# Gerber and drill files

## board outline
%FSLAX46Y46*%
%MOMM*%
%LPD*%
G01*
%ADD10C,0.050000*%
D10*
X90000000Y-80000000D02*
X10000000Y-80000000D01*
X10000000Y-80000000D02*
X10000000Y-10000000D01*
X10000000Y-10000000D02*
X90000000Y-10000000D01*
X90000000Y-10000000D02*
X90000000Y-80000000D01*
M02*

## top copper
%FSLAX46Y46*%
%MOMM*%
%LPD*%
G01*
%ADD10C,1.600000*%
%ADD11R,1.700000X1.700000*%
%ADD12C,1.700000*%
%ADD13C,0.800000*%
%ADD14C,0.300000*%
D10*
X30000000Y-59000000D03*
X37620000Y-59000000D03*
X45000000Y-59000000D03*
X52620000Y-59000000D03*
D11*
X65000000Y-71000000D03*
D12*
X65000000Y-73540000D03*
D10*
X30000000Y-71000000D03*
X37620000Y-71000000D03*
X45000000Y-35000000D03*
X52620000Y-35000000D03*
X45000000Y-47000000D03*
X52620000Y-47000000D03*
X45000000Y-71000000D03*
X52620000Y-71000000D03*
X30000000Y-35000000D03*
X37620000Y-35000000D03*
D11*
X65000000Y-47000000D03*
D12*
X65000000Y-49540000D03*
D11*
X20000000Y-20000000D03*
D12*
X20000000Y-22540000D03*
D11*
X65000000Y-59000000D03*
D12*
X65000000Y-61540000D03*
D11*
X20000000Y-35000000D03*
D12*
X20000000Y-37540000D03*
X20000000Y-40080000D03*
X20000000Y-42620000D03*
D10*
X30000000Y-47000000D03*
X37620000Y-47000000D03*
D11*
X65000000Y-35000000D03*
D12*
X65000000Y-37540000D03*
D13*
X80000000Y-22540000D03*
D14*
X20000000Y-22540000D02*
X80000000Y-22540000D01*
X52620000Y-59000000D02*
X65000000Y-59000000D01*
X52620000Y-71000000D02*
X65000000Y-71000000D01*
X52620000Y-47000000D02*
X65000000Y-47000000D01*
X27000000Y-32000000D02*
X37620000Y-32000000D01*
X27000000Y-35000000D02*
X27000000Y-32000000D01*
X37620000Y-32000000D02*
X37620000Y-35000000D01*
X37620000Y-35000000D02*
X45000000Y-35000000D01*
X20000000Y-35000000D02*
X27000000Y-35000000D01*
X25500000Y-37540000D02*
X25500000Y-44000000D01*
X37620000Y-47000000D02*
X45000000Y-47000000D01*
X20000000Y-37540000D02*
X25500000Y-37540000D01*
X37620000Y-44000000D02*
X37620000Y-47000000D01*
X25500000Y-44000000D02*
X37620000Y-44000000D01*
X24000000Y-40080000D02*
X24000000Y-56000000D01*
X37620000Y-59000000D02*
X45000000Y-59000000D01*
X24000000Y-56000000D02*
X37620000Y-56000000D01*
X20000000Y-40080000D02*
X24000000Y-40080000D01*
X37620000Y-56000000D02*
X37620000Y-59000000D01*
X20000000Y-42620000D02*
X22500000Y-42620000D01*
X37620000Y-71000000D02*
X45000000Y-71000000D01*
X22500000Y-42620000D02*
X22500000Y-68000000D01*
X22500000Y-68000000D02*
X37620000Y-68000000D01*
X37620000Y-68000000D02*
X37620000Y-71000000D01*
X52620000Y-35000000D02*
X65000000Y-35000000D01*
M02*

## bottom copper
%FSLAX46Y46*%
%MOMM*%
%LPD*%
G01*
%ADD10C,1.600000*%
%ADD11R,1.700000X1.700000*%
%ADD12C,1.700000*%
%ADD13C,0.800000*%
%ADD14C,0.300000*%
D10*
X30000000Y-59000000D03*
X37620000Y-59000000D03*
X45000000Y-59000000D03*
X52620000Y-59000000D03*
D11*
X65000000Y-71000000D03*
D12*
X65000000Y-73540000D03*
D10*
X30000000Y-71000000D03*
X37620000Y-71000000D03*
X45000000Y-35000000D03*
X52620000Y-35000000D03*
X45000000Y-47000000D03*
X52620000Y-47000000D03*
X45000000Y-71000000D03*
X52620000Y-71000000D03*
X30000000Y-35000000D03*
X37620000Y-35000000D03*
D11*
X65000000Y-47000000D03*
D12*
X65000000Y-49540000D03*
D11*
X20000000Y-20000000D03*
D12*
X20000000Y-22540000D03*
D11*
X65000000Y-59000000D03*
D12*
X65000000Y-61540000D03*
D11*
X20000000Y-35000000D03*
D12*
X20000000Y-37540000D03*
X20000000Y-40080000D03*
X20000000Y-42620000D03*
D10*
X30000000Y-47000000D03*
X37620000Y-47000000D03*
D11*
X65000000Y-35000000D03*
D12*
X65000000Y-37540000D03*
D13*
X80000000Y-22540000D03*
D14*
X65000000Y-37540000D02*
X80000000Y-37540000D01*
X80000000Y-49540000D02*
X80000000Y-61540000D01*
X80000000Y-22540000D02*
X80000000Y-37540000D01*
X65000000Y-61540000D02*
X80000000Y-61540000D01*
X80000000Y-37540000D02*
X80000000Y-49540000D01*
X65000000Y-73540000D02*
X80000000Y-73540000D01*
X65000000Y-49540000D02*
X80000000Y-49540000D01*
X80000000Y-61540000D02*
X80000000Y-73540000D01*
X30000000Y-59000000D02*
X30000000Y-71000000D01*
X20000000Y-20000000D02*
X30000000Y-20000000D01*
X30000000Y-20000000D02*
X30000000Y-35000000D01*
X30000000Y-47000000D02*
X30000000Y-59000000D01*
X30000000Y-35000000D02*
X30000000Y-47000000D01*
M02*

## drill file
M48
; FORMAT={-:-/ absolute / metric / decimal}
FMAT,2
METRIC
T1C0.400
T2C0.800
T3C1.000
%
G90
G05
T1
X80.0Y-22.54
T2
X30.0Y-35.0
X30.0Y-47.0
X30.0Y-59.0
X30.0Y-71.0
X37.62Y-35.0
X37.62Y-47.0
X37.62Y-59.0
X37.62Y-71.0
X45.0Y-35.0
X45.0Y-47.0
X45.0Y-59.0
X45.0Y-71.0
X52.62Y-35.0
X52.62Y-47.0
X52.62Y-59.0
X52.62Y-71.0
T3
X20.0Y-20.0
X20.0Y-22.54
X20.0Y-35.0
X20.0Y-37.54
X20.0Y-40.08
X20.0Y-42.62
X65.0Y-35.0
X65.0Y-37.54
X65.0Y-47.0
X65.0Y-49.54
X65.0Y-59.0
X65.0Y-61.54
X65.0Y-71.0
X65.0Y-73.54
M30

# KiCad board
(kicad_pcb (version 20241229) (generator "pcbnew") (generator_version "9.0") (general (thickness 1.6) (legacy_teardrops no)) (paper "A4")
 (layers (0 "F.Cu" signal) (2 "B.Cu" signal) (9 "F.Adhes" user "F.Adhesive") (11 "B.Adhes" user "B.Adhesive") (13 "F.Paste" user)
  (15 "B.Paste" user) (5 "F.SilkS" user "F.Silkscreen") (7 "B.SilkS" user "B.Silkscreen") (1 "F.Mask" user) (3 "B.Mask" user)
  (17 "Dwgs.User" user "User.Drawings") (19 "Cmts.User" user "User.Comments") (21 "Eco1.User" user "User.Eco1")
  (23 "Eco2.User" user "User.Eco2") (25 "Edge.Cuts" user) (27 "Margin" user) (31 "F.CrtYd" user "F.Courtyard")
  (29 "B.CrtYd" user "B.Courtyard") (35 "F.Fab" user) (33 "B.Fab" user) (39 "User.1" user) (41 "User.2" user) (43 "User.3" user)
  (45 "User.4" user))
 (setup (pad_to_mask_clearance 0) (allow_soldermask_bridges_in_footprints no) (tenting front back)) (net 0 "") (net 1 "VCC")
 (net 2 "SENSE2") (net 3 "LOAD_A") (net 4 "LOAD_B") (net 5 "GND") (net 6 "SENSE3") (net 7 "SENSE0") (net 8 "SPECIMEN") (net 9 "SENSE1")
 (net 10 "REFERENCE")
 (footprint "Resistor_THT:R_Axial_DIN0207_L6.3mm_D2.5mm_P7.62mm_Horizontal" (layer "F.Cu") (at 30 59)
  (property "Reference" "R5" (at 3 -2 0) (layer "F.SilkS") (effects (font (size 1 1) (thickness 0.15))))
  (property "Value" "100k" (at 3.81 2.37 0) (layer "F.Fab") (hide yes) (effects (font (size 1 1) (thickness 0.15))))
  (pad "1" thru_hole circle (at 0 0) (size 1.6 1.6) (drill 0.8) (layers "*.Cu" "*.Mask") (remove_unused_layers no) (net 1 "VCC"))
  (pad "2" thru_hole circle (at 7.62 0) (size 1.6 1.6) (drill 0.8) (layers "*.Cu" "*.Mask") (remove_unused_layers no) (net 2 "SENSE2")))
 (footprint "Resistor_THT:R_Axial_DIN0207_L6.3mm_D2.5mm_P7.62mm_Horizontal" (layer "F.Cu") (at 45 59)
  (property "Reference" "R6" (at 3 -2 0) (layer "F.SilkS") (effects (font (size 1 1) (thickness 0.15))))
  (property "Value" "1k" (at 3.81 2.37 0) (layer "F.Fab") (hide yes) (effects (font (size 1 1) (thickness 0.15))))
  (pad "1" thru_hole circle (at 0 0) (size 1.6 1.6) (drill 0.8) (layers "*.Cu" "*.Mask") (remove_unused_layers no) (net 2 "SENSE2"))
  (pad "2" thru_hole circle (at 7.62 0) (size 1.6 1.6) (drill 0.8) (layers "*.Cu" "*.Mask") (remove_unused_layers no) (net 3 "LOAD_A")))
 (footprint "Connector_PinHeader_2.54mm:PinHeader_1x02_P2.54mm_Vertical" (layer "F.Cu") (at 65 71)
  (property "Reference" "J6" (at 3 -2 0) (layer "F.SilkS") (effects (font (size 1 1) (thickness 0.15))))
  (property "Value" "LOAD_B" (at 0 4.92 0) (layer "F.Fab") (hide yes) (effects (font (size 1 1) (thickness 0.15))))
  (pad "1" thru_hole rect (at 0 0) (size 1.7 1.7) (drill 1) (layers "*.Cu" "*.Mask") (remove_unused_layers no) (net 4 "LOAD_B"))
  (pad "2" thru_hole circle (at 0 2.54) (size 1.7 1.7) (drill 1) (layers "*.Cu" "*.Mask") (remove_unused_layers no) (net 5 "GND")))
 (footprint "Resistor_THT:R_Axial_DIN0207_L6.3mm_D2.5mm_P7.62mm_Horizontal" (layer "F.Cu") (at 30 71)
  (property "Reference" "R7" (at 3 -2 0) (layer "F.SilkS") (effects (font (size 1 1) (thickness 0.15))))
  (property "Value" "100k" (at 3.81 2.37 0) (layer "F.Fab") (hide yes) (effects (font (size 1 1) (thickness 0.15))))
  (pad "1" thru_hole circle (at 0 0) (size 1.6 1.6) (drill 0.8) (layers "*.Cu" "*.Mask") (remove_unused_layers no) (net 1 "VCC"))
  (pad "2" thru_hole circle (at 7.62 0) (size 1.6 1.6) (drill 0.8) (layers "*.Cu" "*.Mask") (remove_unused_layers no) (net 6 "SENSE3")))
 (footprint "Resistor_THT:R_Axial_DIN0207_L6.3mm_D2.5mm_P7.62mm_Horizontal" (layer "F.Cu") (at 45 35)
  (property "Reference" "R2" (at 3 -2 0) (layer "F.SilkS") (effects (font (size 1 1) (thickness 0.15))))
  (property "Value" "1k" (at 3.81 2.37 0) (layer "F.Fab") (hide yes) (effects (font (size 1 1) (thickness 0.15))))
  (pad "1" thru_hole circle (at 0 0) (size 1.6 1.6) (drill 0.8) (layers "*.Cu" "*.Mask") (remove_unused_layers no) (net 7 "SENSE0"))
  (pad "2" thru_hole circle (at 7.62 0) (size 1.6 1.6) (drill 0.8) (layers "*.Cu" "*.Mask") (remove_unused_layers no) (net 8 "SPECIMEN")))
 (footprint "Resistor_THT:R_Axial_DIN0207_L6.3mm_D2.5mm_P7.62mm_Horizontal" (layer "F.Cu") (at 45 47)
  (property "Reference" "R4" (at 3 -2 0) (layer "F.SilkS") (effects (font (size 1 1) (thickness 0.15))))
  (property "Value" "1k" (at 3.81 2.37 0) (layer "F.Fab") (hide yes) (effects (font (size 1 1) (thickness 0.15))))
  (pad "1" thru_hole circle (at 0 0) (size 1.6 1.6) (drill 0.8) (layers "*.Cu" "*.Mask") (remove_unused_layers no) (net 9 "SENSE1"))
  (pad "2" thru_hole circle (at 7.62 0) (size 1.6 1.6) (drill 0.8) (layers "*.Cu" "*.Mask") (remove_unused_layers no) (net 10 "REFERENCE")))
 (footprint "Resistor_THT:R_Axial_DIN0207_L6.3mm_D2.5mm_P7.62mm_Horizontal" (layer "F.Cu") (at 45 71)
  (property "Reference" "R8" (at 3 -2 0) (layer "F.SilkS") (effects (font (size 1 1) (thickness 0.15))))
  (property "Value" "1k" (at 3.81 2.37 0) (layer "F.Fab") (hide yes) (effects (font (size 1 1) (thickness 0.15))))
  (pad "1" thru_hole circle (at 0 0) (size 1.6 1.6) (drill 0.8) (layers "*.Cu" "*.Mask") (remove_unused_layers no) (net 6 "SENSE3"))
  (pad "2" thru_hole circle (at 7.62 0) (size 1.6 1.6) (drill 0.8) (layers "*.Cu" "*.Mask") (remove_unused_layers no) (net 4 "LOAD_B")))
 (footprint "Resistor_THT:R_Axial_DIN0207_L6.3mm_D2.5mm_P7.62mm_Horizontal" (layer "F.Cu") (at 30 35)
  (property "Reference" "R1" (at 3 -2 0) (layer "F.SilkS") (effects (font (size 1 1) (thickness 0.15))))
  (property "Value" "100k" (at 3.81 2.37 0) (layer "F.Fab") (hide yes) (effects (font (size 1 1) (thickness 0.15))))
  (pad "1" thru_hole circle (at 0 0) (size 1.6 1.6) (drill 0.8) (layers "*.Cu" "*.Mask") (remove_unused_layers no) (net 1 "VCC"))
  (pad "2" thru_hole circle (at 7.62 0) (size 1.6 1.6) (drill 0.8) (layers "*.Cu" "*.Mask") (remove_unused_layers no) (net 7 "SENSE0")))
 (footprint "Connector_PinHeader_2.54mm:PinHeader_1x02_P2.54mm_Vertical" (layer "F.Cu") (at 65 47)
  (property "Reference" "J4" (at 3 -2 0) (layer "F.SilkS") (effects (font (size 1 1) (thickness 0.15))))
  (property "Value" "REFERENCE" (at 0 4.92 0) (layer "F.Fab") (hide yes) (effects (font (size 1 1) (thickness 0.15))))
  (pad "1" thru_hole rect (at 0 0) (size 1.7 1.7) (drill 1) (layers "*.Cu" "*.Mask") (remove_unused_layers no) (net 10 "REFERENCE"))
  (pad "2" thru_hole circle (at 0 2.54) (size 1.7 1.7) (drill 1) (layers "*.Cu" "*.Mask") (remove_unused_layers no) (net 5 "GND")))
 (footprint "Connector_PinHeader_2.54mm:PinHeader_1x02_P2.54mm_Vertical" (layer "F.Cu") (at 20 20)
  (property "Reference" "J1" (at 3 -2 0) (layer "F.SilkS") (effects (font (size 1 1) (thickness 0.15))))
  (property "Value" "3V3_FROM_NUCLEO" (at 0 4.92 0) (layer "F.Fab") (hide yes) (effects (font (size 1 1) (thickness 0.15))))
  (pad "1" thru_hole rect (at 0 0) (size 1.7 1.7) (drill 1) (layers "*.Cu" "*.Mask") (remove_unused_layers no) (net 1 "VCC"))
  (pad "2" thru_hole circle (at 0 2.54) (size 1.7 1.7) (drill 1) (layers "*.Cu" "*.Mask") (remove_unused_layers no) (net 5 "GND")))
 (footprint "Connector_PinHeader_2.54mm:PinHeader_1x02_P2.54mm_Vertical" (layer "F.Cu") (at 65 59)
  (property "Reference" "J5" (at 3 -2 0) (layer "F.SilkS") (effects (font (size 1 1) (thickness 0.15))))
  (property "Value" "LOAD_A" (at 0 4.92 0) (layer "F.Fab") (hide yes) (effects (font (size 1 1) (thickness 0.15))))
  (pad "1" thru_hole rect (at 0 0) (size 1.7 1.7) (drill 1) (layers "*.Cu" "*.Mask") (remove_unused_layers no) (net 3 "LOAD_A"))
  (pad "2" thru_hole circle (at 0 2.54) (size 1.7 1.7) (drill 1) (layers "*.Cu" "*.Mask") (remove_unused_layers no) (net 5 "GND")))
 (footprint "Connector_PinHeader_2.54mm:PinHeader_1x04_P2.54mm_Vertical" (layer "F.Cu") (at 20 35)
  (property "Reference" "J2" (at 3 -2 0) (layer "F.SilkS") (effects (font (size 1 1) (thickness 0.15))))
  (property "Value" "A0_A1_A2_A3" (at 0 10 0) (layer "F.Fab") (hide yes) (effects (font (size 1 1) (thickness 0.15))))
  (pad "1" thru_hole rect (at 0 0) (size 1.7 1.7) (drill 1) (layers "*.Cu" "*.Mask") (remove_unused_layers no) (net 7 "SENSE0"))
  (pad "2" thru_hole circle (at 0 2.54) (size 1.7 1.7) (drill 1) (layers "*.Cu" "*.Mask") (remove_unused_layers no) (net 9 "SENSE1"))
  (pad "3" thru_hole circle (at 0 5.08) (size 1.7 1.7) (drill 1) (layers "*.Cu" "*.Mask") (remove_unused_layers no) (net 2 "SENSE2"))
  (pad "4" thru_hole circle (at 0 7.62) (size 1.7 1.7) (drill 1) (layers "*.Cu" "*.Mask") (remove_unused_layers no) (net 6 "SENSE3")))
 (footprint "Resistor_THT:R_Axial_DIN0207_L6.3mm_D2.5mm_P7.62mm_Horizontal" (layer "F.Cu") (at 30 47)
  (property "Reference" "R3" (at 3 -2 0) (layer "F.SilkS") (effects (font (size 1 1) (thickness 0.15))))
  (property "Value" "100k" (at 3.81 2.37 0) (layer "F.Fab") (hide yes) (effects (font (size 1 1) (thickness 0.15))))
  (pad "1" thru_hole circle (at 0 0) (size 1.6 1.6) (drill 0.8) (layers "*.Cu" "*.Mask") (remove_unused_layers no) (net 1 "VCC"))
  (pad "2" thru_hole circle (at 7.62 0) (size 1.6 1.6) (drill 0.8) (layers "*.Cu" "*.Mask") (remove_unused_layers no) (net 9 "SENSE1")))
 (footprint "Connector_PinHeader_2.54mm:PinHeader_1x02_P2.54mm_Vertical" (layer "F.Cu") (at 65 35)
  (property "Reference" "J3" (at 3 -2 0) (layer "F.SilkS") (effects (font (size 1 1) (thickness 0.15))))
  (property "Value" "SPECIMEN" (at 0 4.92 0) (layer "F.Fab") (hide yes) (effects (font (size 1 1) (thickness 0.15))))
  (pad "1" thru_hole rect (at 0 0) (size 1.7 1.7) (drill 1) (layers "*.Cu" "*.Mask") (remove_unused_layers no) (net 8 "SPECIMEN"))
  (pad "2" thru_hole circle (at 0 2.54) (size 1.7 1.7) (drill 1) (layers "*.Cu" "*.Mask") (remove_unused_layers no) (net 5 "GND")))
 (gr_line (start 90 80) (end 10 80) (stroke (width 0.05) (type default)) (layer "Edge.Cuts"))
 (gr_line (start 10 80) (end 10 10) (stroke (width 0.05) (type default)) (layer "Edge.Cuts"))
 (gr_line (start 10 10) (end 90 10) (stroke (width 0.05) (type default)) (layer "Edge.Cuts"))
 (gr_line (start 90 10) (end 90 80) (stroke (width 0.05) (type default)) (layer "Edge.Cuts"))
 (segment (start 20 22.54) (end 80 22.54) (width 0.3) (layer "F.Cu") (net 5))
 (via (at 80 22.54) (size 0.8) (drill 0.4) (layers "F.Cu" "B.Cu") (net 5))
 (segment (start 65 37.54) (end 80 37.54) (width 0.3) (layer "B.Cu") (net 5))
 (segment (start 80 49.54) (end 80 61.54) (width 0.3) (layer "B.Cu") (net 5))
 (segment (start 80 22.54) (end 80 37.54) (width 0.3) (layer "B.Cu") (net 5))
 (segment (start 65 61.54) (end 80 61.54) (width 0.3) (layer "B.Cu") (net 5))
 (segment (start 80 37.54) (end 80 49.54) (width 0.3) (layer "B.Cu") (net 5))
 (segment (start 65 73.54) (end 80 73.54) (width 0.3) (layer "B.Cu") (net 5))
 (segment (start 65 49.54) (end 80 49.54) (width 0.3) (layer "B.Cu") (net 5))
 (segment (start 80 61.54) (end 80 73.54) (width 0.3) (layer "B.Cu") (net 5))
 (segment (start 52.62 59) (end 65 59) (width 0.3) (layer "F.Cu") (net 3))
 (segment (start 52.62 71) (end 65 71) (width 0.3) (layer "F.Cu") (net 4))
 (segment (start 52.62 47) (end 65 47) (width 0.3) (layer "F.Cu") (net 10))
 (segment (start 27 32) (end 37.62 32) (width 0.3) (layer "F.Cu") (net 7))
 (segment (start 27 35) (end 27 32) (width 0.3) (layer "F.Cu") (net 7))
 (segment (start 37.62 32) (end 37.62 35) (width 0.3) (layer "F.Cu") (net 7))
 (segment (start 37.62 35) (end 45 35) (width 0.3) (layer "F.Cu") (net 7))
 (segment (start 20 35) (end 27 35) (width 0.3) (layer "F.Cu") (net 7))
 (segment (start 25.5 37.54) (end 25.5 44) (width 0.3) (layer "F.Cu") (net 9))
 (segment (start 37.62 47) (end 45 47) (width 0.3) (layer "F.Cu") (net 9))
 (segment (start 20 37.54) (end 25.5 37.54) (width 0.3) (layer "F.Cu") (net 9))
 (segment (start 37.62 44) (end 37.62 47) (width 0.3) (layer "F.Cu") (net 9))
 (segment (start 25.5 44) (end 37.62 44) (width 0.3) (layer "F.Cu") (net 9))
 (segment (start 24 40.08) (end 24 56) (width 0.3) (layer "F.Cu") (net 2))
 (segment (start 37.62 59) (end 45 59) (width 0.3) (layer "F.Cu") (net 2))
 (segment (start 24 56) (end 37.62 56) (width 0.3) (layer "F.Cu") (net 2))
 (segment (start 20 40.08) (end 24 40.08) (width 0.3) (layer "F.Cu") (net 2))
 (segment (start 37.62 56) (end 37.62 59) (width 0.3) (layer "F.Cu") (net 2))
 (segment (start 20 42.62) (end 22.5 42.62) (width 0.3) (layer "F.Cu") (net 6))
 (segment (start 37.62 71) (end 45 71) (width 0.3) (layer "F.Cu") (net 6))
 (segment (start 22.5 42.62) (end 22.5 68) (width 0.3) (layer "F.Cu") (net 6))
 (segment (start 22.5 68) (end 37.62 68) (width 0.3) (layer "F.Cu") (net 6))
 (segment (start 37.62 68) (end 37.62 71) (width 0.3) (layer "F.Cu") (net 6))
 (segment (start 52.62 35) (end 65 35) (width 0.3) (layer "F.Cu") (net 8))
 (segment (start 30 59) (end 30 71) (width 0.3) (layer "B.Cu") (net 1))
 (segment (start 20 20) (end 30 20) (width 0.3) (layer "B.Cu") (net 1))
 (segment (start 30 20) (end 30 35) (width 0.3) (layer "B.Cu") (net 1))
 (segment (start 30 47) (end 30 59) (width 0.3) (layer "B.Cu") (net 1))
 (segment (start 30 35) (end 30 47) (width 0.3) (layer "B.Cu") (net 1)))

